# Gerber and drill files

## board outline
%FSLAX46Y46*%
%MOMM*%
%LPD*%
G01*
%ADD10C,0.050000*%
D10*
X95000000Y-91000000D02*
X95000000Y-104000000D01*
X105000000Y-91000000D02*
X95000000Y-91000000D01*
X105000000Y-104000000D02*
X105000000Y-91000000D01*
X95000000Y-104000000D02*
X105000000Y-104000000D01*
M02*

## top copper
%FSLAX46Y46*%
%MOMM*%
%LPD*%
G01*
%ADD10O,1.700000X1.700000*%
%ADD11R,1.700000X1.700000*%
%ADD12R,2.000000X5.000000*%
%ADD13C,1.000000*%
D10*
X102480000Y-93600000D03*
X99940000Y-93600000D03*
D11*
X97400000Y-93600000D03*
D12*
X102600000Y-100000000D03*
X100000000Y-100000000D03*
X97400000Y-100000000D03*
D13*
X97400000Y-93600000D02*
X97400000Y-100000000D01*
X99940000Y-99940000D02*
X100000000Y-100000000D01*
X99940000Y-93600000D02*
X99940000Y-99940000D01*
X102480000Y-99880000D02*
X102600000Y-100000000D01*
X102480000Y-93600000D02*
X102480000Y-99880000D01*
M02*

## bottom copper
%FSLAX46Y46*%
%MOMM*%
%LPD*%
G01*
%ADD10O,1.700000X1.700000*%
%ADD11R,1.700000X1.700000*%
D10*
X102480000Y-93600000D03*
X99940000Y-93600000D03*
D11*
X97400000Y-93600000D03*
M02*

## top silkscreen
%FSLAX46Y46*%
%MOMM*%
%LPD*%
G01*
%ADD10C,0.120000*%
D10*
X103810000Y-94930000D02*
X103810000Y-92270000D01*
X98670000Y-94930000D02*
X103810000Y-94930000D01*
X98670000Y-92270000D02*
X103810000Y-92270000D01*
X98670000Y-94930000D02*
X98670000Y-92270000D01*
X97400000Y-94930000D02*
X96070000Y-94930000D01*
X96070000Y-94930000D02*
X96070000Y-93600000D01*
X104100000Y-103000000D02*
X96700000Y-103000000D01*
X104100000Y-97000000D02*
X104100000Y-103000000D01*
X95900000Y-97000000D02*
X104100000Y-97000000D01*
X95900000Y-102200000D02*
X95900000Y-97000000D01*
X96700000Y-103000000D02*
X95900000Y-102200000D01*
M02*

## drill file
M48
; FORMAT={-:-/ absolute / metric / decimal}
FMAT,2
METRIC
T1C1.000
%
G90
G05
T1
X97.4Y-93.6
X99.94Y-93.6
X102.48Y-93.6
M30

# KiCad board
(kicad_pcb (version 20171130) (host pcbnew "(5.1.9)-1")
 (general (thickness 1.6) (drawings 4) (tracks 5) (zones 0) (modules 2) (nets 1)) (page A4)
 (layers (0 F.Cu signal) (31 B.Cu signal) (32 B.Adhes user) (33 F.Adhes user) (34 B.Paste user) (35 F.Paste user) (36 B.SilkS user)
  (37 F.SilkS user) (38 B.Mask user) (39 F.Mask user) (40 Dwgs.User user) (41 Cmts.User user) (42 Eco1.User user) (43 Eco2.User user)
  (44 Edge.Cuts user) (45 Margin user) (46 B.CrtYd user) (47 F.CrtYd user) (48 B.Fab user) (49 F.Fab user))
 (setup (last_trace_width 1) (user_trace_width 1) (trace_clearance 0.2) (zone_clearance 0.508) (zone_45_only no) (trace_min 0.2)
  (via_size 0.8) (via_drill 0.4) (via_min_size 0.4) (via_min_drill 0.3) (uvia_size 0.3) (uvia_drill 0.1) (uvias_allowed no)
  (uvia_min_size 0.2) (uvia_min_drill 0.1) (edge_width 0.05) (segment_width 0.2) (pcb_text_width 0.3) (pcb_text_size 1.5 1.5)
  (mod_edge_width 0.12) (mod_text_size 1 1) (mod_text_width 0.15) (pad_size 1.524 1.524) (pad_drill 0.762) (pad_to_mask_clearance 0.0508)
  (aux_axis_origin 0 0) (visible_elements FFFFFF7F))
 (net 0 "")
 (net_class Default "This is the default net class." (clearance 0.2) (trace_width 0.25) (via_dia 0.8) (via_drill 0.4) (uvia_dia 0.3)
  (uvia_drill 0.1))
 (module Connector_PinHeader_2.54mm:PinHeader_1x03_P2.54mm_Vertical (layer F.Cu) (at 97.4 93.6 90)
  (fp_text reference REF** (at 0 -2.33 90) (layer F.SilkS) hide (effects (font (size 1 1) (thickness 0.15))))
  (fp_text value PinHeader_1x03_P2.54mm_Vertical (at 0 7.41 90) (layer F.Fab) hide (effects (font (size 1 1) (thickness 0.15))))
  (fp_line (start -1.33 6.41) (end 1.33 6.41) (layer F.SilkS) (width 0.12))
  (fp_line (start -1.33 1.27) (end -1.33 6.41) (layer F.SilkS) (width 0.12))
  (fp_line (start 1.33 1.27) (end 1.33 6.41) (layer F.SilkS) (width 0.12))
  (fp_line (start -1.33 1.27) (end 1.33 1.27) (layer F.SilkS) (width 0.12))
  (fp_line (start -1.33 0) (end -1.33 -1.33) (layer F.SilkS) (width 0.12))
  (fp_line (start -1.33 -1.33) (end 0 -1.33) (layer F.SilkS) (width 0.12))
  (pad 3 thru_hole oval (at 0 5.08 90) (size 1.7 1.7) (drill 1) (layers *.Cu *.Mask))
  (pad 2 thru_hole oval (at 0 2.54 90) (size 1.7 1.7) (drill 1) (layers *.Cu *.Mask))
  (pad 1 thru_hole rect (at 0 0 90) (size 1.7 1.7) (drill 1) (layers *.Cu *.Mask)))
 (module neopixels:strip (layer F.Cu) (at 100 100)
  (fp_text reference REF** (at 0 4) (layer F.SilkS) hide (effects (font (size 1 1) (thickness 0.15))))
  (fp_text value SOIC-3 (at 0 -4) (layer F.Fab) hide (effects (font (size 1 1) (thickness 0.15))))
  (fp_line (start 4.1 3) (end -3.3 3) (layer F.SilkS) (width 0.12))
  (fp_line (start 4.1 -3) (end 4.1 3) (layer F.SilkS) (width 0.12))
  (fp_line (start -4.1 -3) (end 4.1 -3) (layer F.SilkS) (width 0.12))
  (fp_line (start -4.1 2.2) (end -4.1 -3) (layer F.SilkS) (width 0.12))
  (fp_line (start -3.3 3) (end -4.1 2.2) (layer F.SilkS) (width 0.12))
  (pad 3 smd rect (at 2.6 0) (size 2 5) (layers F.Cu F.Paste F.Mask))
  (pad 2 smd rect (at 0 0) (size 2 5) (layers F.Cu F.Paste F.Mask))
  (pad 1 smd rect (at -2.6 0) (size 2 5) (layers F.Cu F.Paste F.Mask)))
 (gr_line (start 95 91) (end 95 104) (layer Edge.Cuts) (width 0.05))
 (gr_line (start 105 91) (end 95 91) (layer Edge.Cuts) (width 0.05))
 (gr_line (start 105 104) (end 105 91) (layer Edge.Cuts) (width 0.05))
 (gr_line (start 95 104) (end 105 104) (layer Edge.Cuts) (width 0.05))
 (segment (start 97.4 93.6) (end 97.4 100) (width 1) (layer F.Cu) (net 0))
 (segment (start 99.94 99.94) (end 100 100) (width 1) (layer F.Cu) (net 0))
 (segment (start 99.94 93.6) (end 99.94 99.94) (width 1) (layer F.Cu) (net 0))
 (segment (start 102.48 99.88) (end 102.6 100) (width 1) (layer F.Cu) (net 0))
 (segment (start 102.48 93.6) (end 102.48 99.88) (width 1) (layer F.Cu) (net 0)))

